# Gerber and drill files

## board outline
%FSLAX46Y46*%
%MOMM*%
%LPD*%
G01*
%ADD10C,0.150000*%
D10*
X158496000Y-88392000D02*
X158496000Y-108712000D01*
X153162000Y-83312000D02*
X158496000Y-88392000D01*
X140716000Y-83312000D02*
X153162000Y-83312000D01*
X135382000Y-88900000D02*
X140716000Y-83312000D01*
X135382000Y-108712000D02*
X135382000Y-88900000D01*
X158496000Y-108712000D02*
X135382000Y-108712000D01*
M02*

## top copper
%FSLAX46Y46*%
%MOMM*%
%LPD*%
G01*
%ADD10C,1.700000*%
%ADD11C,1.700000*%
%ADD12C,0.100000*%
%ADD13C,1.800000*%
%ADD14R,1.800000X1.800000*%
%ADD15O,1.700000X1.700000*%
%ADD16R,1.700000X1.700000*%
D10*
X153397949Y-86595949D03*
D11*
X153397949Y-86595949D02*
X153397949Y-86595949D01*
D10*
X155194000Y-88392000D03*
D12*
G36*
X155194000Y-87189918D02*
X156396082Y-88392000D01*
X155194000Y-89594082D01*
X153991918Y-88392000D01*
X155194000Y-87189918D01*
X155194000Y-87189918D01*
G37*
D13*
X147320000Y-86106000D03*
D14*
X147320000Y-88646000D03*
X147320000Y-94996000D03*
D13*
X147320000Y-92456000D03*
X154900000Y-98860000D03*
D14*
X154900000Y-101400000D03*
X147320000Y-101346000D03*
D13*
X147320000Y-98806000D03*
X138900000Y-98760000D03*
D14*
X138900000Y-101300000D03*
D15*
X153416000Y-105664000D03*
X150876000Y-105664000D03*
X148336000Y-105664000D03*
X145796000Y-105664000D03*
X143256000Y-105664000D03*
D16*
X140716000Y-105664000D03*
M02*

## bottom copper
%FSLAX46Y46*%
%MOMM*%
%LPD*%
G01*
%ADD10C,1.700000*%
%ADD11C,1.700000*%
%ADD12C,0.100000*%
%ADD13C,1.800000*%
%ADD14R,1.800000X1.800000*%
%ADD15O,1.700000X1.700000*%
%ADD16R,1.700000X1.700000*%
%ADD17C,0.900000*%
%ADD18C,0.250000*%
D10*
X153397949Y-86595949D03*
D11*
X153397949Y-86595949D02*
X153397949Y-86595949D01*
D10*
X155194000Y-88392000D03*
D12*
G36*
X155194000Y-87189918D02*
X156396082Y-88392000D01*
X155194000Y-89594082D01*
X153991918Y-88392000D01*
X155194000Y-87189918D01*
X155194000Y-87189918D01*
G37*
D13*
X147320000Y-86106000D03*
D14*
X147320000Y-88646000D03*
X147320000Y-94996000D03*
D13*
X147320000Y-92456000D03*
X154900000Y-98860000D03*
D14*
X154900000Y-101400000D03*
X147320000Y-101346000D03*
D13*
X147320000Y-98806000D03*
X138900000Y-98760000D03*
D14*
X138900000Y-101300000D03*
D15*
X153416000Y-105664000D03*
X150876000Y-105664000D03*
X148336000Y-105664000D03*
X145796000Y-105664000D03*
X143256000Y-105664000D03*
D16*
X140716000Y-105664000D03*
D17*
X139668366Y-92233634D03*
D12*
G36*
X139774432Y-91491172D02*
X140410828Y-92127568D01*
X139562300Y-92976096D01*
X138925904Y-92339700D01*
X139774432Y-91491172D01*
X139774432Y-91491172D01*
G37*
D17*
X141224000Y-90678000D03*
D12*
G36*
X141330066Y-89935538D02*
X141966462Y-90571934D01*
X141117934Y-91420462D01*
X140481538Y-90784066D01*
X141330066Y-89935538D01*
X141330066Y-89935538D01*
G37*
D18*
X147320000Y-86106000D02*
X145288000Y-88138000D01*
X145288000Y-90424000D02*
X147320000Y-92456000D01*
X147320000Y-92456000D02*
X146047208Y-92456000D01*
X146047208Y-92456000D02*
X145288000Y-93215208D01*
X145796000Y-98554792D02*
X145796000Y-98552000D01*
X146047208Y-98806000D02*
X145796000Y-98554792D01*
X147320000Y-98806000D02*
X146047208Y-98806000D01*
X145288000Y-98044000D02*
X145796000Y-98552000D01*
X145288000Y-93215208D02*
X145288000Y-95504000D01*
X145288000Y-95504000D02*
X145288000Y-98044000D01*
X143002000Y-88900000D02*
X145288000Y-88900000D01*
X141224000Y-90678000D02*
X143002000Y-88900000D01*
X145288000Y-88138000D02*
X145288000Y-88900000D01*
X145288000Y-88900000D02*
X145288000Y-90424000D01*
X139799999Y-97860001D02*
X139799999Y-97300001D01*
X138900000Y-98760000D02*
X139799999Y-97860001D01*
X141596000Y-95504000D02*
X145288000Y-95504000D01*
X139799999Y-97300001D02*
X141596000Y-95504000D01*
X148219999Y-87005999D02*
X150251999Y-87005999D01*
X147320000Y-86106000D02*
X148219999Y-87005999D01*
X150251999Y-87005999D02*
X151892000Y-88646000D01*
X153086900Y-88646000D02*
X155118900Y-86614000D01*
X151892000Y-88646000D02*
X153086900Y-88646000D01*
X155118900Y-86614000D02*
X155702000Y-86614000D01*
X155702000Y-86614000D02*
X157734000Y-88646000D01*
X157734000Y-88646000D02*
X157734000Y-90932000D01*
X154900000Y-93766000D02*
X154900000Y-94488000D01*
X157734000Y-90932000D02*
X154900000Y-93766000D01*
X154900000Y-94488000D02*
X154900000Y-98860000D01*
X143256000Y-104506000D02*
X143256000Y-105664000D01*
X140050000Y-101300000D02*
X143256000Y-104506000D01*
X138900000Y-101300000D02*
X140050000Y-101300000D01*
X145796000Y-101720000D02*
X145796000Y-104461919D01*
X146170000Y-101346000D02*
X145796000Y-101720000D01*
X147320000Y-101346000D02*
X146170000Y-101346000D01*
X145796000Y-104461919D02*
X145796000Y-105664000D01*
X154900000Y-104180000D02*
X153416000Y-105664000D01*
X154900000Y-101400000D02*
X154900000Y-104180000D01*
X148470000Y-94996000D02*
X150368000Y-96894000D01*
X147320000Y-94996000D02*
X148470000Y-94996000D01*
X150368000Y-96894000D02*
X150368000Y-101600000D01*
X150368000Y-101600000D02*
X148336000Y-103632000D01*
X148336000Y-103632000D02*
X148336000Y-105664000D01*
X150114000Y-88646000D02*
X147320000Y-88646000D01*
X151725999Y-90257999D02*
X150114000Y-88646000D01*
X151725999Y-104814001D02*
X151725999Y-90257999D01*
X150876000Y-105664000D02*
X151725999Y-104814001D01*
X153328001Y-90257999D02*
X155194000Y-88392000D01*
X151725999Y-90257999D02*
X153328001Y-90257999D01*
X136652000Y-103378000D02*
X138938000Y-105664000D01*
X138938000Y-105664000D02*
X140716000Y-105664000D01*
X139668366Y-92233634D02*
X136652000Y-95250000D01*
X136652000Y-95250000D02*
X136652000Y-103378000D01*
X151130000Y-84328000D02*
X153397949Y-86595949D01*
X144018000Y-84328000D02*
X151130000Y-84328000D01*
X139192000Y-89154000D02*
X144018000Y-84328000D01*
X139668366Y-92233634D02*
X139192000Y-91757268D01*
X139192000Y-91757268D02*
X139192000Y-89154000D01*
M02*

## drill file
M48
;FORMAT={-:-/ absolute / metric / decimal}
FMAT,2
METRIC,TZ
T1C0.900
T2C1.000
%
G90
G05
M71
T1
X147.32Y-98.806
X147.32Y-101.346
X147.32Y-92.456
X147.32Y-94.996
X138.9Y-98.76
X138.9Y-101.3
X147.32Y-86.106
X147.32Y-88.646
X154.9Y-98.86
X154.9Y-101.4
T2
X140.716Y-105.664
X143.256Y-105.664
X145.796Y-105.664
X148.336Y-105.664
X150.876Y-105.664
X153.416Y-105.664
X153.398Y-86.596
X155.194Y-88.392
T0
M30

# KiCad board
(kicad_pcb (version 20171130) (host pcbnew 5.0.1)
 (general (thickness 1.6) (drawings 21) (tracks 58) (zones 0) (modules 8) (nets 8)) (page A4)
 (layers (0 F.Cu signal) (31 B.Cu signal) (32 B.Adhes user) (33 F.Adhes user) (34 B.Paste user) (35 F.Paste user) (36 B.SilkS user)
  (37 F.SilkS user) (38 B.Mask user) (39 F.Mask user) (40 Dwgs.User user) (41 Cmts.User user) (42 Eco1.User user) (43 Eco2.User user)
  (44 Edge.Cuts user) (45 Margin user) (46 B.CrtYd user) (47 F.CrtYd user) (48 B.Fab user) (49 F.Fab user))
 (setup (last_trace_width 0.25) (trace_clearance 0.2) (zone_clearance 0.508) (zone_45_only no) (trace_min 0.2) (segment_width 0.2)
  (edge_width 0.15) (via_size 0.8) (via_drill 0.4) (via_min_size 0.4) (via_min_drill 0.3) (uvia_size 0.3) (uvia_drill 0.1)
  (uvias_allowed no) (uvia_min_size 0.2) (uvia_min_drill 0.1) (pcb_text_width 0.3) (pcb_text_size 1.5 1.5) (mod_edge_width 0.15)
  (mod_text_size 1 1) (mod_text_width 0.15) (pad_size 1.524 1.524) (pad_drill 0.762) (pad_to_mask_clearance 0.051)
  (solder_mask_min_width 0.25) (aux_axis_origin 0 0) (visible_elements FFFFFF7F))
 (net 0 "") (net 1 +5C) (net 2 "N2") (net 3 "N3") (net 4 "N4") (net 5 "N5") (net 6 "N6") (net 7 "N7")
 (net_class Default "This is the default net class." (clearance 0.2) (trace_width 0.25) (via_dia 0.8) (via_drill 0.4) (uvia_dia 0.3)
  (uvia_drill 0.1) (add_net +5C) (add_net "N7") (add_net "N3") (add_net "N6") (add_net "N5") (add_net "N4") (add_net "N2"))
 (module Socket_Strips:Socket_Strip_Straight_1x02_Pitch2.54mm (layer F.Cu) (at 155.194 88.392 225)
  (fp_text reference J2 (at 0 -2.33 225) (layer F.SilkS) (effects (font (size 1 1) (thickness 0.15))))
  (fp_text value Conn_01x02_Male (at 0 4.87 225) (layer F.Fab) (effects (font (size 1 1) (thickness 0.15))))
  (pad 2 thru_hole oval (at 0 2.54 225) (size 1.7 1.7) (drill 1) (layers *.Cu *.Mask) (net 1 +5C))
  (pad 1 thru_hole rect (at 0 0 225) (size 1.7 1.7) (drill 1) (layers *.Cu *.Mask) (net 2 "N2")))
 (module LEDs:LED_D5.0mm (layer F.Cu) (at 147.32 88.646 90)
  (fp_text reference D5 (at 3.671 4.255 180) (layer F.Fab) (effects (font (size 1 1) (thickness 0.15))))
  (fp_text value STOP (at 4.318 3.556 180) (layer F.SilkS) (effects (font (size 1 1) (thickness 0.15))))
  (pad 2 thru_hole circle (at 2.54 0 90) (size 1.8 1.8) (drill 0.9) (layers *.Cu *.Mask) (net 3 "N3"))
  (pad 1 thru_hole rect (at 0 0 90) (size 1.8 1.8) (drill 0.9) (layers *.Cu *.Mask) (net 2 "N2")))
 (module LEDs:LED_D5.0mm (layer F.Cu) (at 147.32 94.996 90)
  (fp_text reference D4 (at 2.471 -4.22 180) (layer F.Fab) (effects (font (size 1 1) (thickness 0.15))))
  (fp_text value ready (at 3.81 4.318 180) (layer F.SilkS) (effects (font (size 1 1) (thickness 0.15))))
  (pad 1 thru_hole rect (at 0 0 90) (size 1.8 1.8) (drill 0.9) (layers *.Cu *.Mask) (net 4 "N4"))
  (pad 2 thru_hole circle (at 2.54 0 90) (size 1.8 1.8) (drill 0.9) (layers *.Cu *.Mask) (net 3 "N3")))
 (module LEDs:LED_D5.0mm (layer F.Cu) (at 154.9 101.4 90)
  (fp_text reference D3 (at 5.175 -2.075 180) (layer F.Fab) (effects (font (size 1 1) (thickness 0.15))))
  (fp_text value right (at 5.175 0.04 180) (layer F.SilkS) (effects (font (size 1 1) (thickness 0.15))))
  (pad 2 thru_hole circle (at 2.54 0 90) (size 1.8 1.8) (drill 0.9) (layers *.Cu *.Mask) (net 3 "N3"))
  (pad 1 thru_hole rect (at 0 0 90) (size 1.8 1.8) (drill 0.9) (layers *.Cu *.Mask) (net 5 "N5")))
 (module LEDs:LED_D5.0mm (layer F.Cu) (at 147.32 101.346 90)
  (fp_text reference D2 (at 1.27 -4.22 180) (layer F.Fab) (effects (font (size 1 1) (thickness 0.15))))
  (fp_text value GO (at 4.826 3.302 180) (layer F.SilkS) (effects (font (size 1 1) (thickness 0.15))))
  (pad 1 thru_hole rect (at 0 0 90) (size 1.8 1.8) (drill 0.9) (layers *.Cu *.Mask) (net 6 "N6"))
  (pad 2 thru_hole circle (at 2.54 0 90) (size 1.8 1.8) (drill 0.9) (layers *.Cu *.Mask) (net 3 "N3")))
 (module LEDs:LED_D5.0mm (layer F.Cu) (at 138.9 101.3 90)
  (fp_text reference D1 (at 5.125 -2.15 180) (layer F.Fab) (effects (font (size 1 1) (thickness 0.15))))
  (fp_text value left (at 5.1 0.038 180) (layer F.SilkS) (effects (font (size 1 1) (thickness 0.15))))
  (pad 2 thru_hole circle (at 2.54 0 90) (size 1.8 1.8) (drill 0.9) (layers *.Cu *.Mask) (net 3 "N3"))
  (pad 1 thru_hole rect (at 0 0 90) (size 1.8 1.8) (drill 0.9) (layers *.Cu *.Mask) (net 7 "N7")))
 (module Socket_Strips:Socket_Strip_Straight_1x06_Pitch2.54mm (layer F.Cu) (at 140.716 105.664 90)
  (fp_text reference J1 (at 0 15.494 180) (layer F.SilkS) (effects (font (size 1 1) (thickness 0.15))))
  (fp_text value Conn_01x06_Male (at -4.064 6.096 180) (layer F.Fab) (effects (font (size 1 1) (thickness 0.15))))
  (pad 6 thru_hole oval (at 0 12.7 90) (size 1.7 1.7) (drill 1) (layers *.Cu *.Mask) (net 5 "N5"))
  (pad 5 thru_hole oval (at 0 10.16 90) (size 1.7 1.7) (drill 1) (layers *.Cu *.Mask) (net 2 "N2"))
  (pad 4 thru_hole oval (at 0 7.62 90) (size 1.7 1.7) (drill 1) (layers *.Cu *.Mask) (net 4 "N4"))
  (pad 3 thru_hole oval (at 0 5.08 90) (size 1.7 1.7) (drill 1) (layers *.Cu *.Mask) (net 6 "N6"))
  (pad 2 thru_hole oval (at 0 2.54 90) (size 1.7 1.7) (drill 1) (layers *.Cu *.Mask) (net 7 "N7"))
  (pad 1 thru_hole rect (at 0 0 90) (size 1.7 1.7) (drill 1) (layers *.Cu *.Mask) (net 1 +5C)))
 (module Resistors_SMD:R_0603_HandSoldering (layer B.Cu) (at 140.446183 91.455817 225)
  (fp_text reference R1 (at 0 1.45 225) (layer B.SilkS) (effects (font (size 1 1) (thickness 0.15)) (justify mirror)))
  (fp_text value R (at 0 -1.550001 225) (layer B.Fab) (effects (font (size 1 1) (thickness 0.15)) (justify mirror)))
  (pad 2 smd rect (at 1.099999 0 225) (size 1.2 0.9) (layers B.Cu B.Paste B.Mask) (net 1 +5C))
  (pad 1 smd rect (at -1.099999 0 225) (size 1.2 0.9) (layers B.Cu B.Paste B.Mask) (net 3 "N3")))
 (gr_line (start 158.496 88.392) (end 158.496 108.712) (layer Edge.Cuts) (width 0.15))
 (gr_line (start 153.162 83.312) (end 158.496 88.392) (layer Edge.Cuts) (width 0.15))
 (gr_line (start 140.716 83.312) (end 153.162 83.312) (layer Edge.Cuts) (width 0.15))
 (gr_line (start 135.382 88.9) (end 140.716 83.312) (layer Edge.Cuts) (width 0.15))
 (gr_line (start 135.382 108.712) (end 135.382 88.9) (layer Edge.Cuts) (width 0.15))
 (gr_line (start 158.496 108.712) (end 135.382 108.712) (layer Edge.Cuts) (width 0.15))
 (segment (start 147.32 86.106) (end 145.288 88.138) (width 0.25) (layer B.Cu) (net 3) (status 10))
 (segment (start 145.288 90.424) (end 147.32 92.456) (width 0.25) (layer B.Cu) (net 3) (status 20))
 (segment (start 147.32 92.456) (end 146.047208 92.456) (width 0.25) (layer B.Cu) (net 3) (status 10))
 (segment (start 146.047208 92.456) (end 145.288 93.215208) (width 0.25) (layer B.Cu) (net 3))
 (segment (start 145.796 98.554792) (end 145.796 98.552) (width 0.25) (layer B.Cu) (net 3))
 (segment (start 146.047208 98.806) (end 145.796 98.554792) (width 0.25) (layer B.Cu) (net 3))
 (segment (start 147.32 98.806) (end 146.047208 98.806) (width 0.25) (layer B.Cu) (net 3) (status 10))
 (segment (start 145.288 98.044) (end 145.796 98.552) (width 0.25) (layer B.Cu) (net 3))
 (segment (start 145.288 93.215208) (end 145.288 95.504) (width 0.25) (layer B.Cu) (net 3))
 (segment (start 145.288 95.504) (end 145.288 98.044) (width 0.25) (layer B.Cu) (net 3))
 (segment (start 143.002 88.9) (end 145.288 88.9) (width 0.25) (layer B.Cu) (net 3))
 (segment (start 141.224 90.678) (end 143.002 88.9) (width 0.25) (layer B.Cu) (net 3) (status 10))
 (segment (start 145.288 88.138) (end 145.288 88.9) (width 0.25) (layer B.Cu) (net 3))
 (segment (start 145.288 88.9) (end 145.288 90.424) (width 0.25) (layer B.Cu) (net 3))
 (segment (start 139.799999 97.860001) (end 139.799999 97.300001) (width 0.25) (layer B.Cu) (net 3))
 (segment (start 138.9 98.76) (end 139.799999 97.860001) (width 0.25) (layer B.Cu) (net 3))
 (segment (start 141.596 95.504) (end 145.288 95.504) (width 0.25) (layer B.Cu) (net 3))
 (segment (start 139.799999 97.300001) (end 141.596 95.504) (width 0.25) (layer B.Cu) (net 3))
 (segment (start 148.219999 87.005999) (end 150.251999 87.005999) (width 0.25) (layer B.Cu) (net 3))
 (segment (start 147.32 86.106) (end 148.219999 87.005999) (width 0.25) (layer B.Cu) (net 3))
 (segment (start 150.251999 87.005999) (end 151.892 88.646) (width 0.25) (layer B.Cu) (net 3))
 (segment (start 153.0869 88.646) (end 155.1189 86.614) (width 0.25) (layer B.Cu) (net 3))
 (segment (start 151.892 88.646) (end 153.0869 88.646) (width 0.25) (layer B.Cu) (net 3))
 (segment (start 155.1189 86.614) (end 155.702 86.614) (width 0.25) (layer B.Cu) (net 3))
 (segment (start 155.702 86.614) (end 157.734 88.646) (width 0.25) (layer B.Cu) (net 3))
 (segment (start 157.734 88.646) (end 157.734 90.932) (width 0.25) (layer B.Cu) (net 3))
 (segment (start 154.9 93.766) (end 154.9 94.488) (width 0.25) (layer B.Cu) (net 3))
 (segment (start 157.734 90.932) (end 154.9 93.766) (width 0.25) (layer B.Cu) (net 3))
 (segment (start 154.9 94.488) (end 154.9 98.86) (width 0.25) (layer B.Cu) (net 3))
 (segment (start 143.256 104.506) (end 143.256 105.664) (width 0.25) (layer B.Cu) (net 7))
 (segment (start 140.05 101.3) (end 143.256 104.506) (width 0.25) (layer B.Cu) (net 7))
 (segment (start 138.9 101.3) (end 140.05 101.3) (width 0.25) (layer B.Cu) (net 7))
 (segment (start 145.796 101.72) (end 145.796 104.461919) (width 0.25) (layer B.Cu) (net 6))
 (segment (start 146.17 101.346) (end 145.796 101.72) (width 0.25) (layer B.Cu) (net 6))
 (segment (start 147.32 101.346) (end 146.17 101.346) (width 0.25) (layer B.Cu) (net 6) (status 10))
 (segment (start 145.796 104.461919) (end 145.796 105.664) (width 0.25) (layer B.Cu) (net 6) (status 20))
 (segment (start 154.9 104.18) (end 153.416 105.664) (width 0.25) (layer B.Cu) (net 5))
 (segment (start 154.9 101.4) (end 154.9 104.18) (width 0.25) (layer B.Cu) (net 5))
 (segment (start 148.47 94.996) (end 150.368 96.894) (width 0.25) (layer B.Cu) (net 4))
 (segment (start 147.32 94.996) (end 148.47 94.996) (width 0.25) (layer B.Cu) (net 4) (status 10))
 (segment (start 150.368 96.894) (end 150.368 101.6) (width 0.25) (layer B.Cu) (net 4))
 (segment (start 150.368 101.6) (end 148.336 103.632) (width 0.25) (layer B.Cu) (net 4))
 (segment (start 148.336 103.632) (end 148.336 105.664) (width 0.25) (layer B.Cu) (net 4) (status 20))
 (segment (start 150.114 88.646) (end 147.32 88.646) (width 0.25) (layer B.Cu) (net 2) (status 20))
 (segment (start 151.725999 90.257999) (end 150.114 88.646) (width 0.25) (layer B.Cu) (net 2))
 (segment (start 151.725999 104.814001) (end 151.725999 90.257999) (width 0.25) (layer B.Cu) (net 2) (status 10))
 (segment (start 150.876 105.664) (end 151.725999 104.814001) (width 0.25) (layer B.Cu) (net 2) (status 30))
 (segment (start 153.328001 90.257999) (end 155.194 88.392) (width 0.25) (layer B.Cu) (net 2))
 (segment (start 151.725999 90.257999) (end 153.328001 90.257999) (width 0.25) (layer B.Cu) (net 2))
 (segment (start 136.652 103.378) (end 138.938 105.664) (width 0.25) (layer B.Cu) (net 1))
 (segment (start 138.938 105.664) (end 140.716 105.664) (width 0.25) (layer B.Cu) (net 1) (status 20))
 (segment (start 139.668366 92.233634) (end 136.652 95.25) (width 0.25) (layer B.Cu) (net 1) (status 10))
 (segment (start 136.652 95.25) (end 136.652 103.378) (width 0.25) (layer B.Cu) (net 1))
 (segment (start 151.13 84.328) (end 153.397949 86.595949) (width 0.25) (layer B.Cu) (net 1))
 (segment (start 144.018 84.328) (end 151.13 84.328) (width 0.25) (layer B.Cu) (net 1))
 (segment (start 139.192 89.154) (end 144.018 84.328) (width 0.25) (layer B.Cu) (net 1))
 (segment (start 139.668366 92.233634) (end 139.192 91.757268) (width 0.25) (layer B.Cu) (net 1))
 (segment (start 139.192 91.757268) (end 139.192 89.154) (width 0.25) (layer B.Cu) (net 1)))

